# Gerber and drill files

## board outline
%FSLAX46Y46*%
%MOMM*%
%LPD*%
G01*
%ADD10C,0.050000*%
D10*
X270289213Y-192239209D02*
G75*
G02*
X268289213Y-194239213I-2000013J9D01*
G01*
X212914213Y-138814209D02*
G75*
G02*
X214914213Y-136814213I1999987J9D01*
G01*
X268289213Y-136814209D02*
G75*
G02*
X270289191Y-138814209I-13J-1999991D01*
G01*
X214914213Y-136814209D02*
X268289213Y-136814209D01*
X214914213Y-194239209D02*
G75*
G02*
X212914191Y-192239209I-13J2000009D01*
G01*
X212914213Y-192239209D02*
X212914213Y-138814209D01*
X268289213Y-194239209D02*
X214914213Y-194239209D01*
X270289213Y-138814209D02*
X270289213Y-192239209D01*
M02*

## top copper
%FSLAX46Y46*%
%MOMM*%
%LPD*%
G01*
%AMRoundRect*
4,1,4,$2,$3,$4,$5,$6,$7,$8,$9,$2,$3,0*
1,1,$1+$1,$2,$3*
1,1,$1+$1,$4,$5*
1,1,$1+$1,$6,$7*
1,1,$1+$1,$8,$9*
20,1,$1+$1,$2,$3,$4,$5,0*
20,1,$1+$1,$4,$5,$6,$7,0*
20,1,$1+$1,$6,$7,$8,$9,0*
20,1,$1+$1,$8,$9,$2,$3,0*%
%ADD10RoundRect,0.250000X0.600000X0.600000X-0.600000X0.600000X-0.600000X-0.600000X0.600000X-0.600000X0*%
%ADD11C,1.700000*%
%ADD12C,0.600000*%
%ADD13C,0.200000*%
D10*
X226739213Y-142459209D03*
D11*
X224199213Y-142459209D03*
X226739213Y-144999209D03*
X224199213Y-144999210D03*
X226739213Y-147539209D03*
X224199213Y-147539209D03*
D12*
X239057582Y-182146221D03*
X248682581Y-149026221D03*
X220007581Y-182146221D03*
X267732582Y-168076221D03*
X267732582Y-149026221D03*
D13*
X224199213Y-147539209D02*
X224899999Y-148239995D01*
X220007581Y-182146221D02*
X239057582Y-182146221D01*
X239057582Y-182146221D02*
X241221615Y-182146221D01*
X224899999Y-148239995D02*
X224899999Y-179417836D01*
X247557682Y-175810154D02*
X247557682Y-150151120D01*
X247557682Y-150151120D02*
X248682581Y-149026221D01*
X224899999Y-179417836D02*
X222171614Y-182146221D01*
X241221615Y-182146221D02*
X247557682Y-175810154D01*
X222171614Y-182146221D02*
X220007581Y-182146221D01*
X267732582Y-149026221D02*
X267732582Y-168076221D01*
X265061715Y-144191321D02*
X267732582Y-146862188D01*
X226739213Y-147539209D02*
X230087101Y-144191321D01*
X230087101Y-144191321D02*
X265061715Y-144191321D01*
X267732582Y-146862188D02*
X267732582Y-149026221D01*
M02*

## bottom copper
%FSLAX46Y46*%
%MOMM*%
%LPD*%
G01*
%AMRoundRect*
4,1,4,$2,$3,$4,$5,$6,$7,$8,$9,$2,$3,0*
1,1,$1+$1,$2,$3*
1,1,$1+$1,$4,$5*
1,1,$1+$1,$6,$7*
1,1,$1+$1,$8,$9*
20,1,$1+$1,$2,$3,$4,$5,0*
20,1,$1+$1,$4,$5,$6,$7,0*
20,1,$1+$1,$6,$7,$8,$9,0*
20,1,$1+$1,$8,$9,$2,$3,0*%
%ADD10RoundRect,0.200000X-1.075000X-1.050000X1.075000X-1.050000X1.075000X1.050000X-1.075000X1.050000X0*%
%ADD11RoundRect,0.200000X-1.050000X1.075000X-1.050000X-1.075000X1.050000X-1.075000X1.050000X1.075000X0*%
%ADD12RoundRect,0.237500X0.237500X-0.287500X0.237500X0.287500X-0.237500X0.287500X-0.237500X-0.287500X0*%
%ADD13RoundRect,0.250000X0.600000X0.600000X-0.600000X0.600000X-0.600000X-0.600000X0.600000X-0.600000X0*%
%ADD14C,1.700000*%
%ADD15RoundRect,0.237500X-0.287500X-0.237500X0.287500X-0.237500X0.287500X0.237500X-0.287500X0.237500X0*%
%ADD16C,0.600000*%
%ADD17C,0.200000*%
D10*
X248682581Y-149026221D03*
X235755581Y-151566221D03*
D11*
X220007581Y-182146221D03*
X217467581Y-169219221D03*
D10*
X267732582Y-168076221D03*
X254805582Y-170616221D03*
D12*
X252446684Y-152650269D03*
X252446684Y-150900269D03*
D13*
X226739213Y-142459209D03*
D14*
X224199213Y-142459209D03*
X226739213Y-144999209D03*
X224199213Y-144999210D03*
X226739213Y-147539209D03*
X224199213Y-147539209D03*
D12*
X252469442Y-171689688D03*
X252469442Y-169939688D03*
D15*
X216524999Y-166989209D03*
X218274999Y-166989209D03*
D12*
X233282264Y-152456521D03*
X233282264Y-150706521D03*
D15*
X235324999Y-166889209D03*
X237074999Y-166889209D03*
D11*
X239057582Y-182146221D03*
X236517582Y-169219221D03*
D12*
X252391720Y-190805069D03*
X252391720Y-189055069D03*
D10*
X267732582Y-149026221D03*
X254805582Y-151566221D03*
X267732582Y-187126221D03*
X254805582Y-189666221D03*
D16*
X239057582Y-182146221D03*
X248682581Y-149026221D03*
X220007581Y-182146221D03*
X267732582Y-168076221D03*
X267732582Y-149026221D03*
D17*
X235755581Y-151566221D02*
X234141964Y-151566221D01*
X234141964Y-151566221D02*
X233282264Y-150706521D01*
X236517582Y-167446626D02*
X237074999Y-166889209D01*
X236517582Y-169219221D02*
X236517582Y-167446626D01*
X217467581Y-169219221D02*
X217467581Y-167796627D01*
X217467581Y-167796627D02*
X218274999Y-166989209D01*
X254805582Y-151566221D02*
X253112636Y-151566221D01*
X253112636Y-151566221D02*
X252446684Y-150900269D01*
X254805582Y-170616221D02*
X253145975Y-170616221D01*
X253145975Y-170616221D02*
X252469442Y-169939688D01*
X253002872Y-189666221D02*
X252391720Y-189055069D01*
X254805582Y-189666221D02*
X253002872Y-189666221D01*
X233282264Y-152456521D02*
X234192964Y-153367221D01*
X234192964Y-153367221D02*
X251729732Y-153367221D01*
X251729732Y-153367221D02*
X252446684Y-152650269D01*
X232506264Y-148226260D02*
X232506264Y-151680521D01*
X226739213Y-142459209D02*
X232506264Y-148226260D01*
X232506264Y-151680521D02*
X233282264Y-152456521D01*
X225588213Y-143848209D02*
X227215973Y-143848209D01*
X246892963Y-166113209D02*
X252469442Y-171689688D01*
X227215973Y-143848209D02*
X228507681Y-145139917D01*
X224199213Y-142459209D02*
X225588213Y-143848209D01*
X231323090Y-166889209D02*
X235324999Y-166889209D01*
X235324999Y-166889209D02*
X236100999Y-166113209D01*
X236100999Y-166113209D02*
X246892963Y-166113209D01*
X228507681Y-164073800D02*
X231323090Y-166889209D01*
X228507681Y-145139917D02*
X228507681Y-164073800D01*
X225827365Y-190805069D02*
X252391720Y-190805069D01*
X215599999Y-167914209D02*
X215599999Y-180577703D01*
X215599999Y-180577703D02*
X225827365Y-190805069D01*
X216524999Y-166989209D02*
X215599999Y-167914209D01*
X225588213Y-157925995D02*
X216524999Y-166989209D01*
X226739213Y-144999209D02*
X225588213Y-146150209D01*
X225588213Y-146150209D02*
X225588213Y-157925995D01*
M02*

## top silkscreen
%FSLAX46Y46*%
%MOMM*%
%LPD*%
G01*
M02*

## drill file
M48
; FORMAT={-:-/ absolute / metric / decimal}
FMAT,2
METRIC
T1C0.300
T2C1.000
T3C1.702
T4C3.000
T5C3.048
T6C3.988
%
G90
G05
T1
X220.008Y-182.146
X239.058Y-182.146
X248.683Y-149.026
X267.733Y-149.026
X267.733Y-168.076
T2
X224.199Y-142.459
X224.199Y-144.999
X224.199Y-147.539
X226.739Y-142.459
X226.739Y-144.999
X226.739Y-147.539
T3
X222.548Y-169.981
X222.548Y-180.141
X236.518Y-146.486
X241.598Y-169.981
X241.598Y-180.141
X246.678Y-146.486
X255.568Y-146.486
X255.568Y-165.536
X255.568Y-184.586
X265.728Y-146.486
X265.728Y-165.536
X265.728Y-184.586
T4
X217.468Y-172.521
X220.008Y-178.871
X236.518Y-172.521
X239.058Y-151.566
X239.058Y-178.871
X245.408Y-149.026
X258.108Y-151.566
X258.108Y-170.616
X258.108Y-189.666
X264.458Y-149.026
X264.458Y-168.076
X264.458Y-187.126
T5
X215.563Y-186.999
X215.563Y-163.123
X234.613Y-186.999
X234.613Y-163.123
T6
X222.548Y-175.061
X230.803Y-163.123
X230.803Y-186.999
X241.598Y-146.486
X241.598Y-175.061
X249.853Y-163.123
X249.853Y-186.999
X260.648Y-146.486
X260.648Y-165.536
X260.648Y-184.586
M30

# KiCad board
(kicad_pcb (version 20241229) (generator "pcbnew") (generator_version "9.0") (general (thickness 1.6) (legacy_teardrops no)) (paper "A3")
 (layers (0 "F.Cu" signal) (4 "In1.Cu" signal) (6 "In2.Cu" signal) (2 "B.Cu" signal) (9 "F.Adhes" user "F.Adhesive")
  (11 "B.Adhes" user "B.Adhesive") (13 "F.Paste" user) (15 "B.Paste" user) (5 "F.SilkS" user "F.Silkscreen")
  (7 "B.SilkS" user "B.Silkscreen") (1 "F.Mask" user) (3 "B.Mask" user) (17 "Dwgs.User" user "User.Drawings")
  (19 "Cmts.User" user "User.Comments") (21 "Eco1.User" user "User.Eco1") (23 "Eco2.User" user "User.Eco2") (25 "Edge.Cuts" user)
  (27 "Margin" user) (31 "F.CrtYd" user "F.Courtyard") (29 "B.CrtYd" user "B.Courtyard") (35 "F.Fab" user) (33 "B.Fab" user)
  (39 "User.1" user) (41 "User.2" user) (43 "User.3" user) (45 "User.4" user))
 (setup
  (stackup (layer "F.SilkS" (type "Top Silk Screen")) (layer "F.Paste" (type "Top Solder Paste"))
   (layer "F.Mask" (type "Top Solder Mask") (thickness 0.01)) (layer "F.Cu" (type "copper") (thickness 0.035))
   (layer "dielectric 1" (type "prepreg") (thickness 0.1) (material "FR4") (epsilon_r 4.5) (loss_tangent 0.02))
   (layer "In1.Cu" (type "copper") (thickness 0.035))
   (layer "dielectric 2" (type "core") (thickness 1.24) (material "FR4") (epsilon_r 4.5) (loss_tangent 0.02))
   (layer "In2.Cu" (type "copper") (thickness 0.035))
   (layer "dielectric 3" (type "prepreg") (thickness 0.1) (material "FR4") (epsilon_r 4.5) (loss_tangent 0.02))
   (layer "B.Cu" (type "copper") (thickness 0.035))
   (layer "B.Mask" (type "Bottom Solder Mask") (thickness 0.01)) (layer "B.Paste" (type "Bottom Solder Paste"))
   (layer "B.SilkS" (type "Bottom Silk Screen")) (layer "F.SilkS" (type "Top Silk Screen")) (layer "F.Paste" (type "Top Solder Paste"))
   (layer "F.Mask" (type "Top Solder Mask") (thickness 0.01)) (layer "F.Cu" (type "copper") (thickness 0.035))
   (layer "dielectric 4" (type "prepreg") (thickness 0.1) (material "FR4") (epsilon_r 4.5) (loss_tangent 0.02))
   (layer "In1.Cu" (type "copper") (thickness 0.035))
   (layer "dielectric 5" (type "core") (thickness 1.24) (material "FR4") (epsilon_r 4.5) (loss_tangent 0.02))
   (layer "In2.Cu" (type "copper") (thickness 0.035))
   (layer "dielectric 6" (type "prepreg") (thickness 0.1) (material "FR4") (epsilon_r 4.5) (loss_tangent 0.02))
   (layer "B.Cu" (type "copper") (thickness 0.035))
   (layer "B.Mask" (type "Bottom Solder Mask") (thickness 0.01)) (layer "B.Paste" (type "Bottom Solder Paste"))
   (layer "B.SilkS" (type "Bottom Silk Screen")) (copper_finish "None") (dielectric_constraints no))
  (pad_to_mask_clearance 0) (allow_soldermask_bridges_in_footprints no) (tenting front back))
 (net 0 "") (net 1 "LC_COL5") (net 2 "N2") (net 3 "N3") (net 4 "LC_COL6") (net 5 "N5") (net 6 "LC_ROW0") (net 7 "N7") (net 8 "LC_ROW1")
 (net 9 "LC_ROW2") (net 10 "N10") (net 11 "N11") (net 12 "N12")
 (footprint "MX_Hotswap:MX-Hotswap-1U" (layer "B.Cu") (at 241.597581 146.486221)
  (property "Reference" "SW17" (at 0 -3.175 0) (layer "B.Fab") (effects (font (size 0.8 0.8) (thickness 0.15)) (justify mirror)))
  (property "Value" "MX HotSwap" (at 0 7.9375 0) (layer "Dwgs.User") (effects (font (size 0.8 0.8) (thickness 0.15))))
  (pad "" np_thru_hole circle (at -5.08 0 48.099) (size 1.7018 1.7018) (drill 1.7018) (layers "*.Cu" "*.Mask"))
  (pad "" np_thru_hole circle (at -2.54 5.08) (size 3 3) (drill 3) (layers "*.Cu" "*.Mask"))
  (pad "" np_thru_hole circle (at 0 0) (size 3.9878 3.9878) (drill 3.9878) (layers "*.Cu" "*.Mask"))
  (pad "" np_thru_hole circle (at 3.81 2.54) (size 3 3) (drill 3) (layers "*.Cu" "*.Mask"))
  (pad "" np_thru_hole circle (at 5.08 0 48.099) (size 1.7018 1.7018) (drill 1.7018) (layers "*.Cu" "*.Mask"))
  (pad "1" smd roundrect (at 7.085 2.54) (size 2.55 2.5) (layers "B.Cu" "B.Mask" "B.Paste") (roundrect_rratio 0.08) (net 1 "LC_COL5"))
  (pad "2" smd roundrect (at -5.842 5.08) (size 2.55 2.5) (layers "B.Cu" "B.Mask" "B.Paste") (roundrect_rratio 0.08) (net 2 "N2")))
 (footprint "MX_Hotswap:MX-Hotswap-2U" (layer "B.Cu") (at 222.547581 175.061221 -90)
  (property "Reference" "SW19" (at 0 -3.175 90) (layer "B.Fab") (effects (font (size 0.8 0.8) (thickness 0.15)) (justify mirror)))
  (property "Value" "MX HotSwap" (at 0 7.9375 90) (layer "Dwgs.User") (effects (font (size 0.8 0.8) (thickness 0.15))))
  (pad "" np_thru_hole circle (at -11.938 -8.255 270) (size 3.9878 3.9878) (drill 3.9878) (layers "*.Cu" "*.Mask"))
  (pad "" np_thru_hole circle (at -11.938 6.984999 270) (size 3.048 3.048) (drill 3.048) (layers "*.Cu" "*.Mask"))
  (pad "" np_thru_hole circle (at -5.08 0 318.099) (size 1.7018 1.7018) (drill 1.7018) (layers "*.Cu" "*.Mask"))
  (pad "" np_thru_hole circle (at -2.54 5.08 270) (size 3 3) (drill 3) (layers "*.Cu" "*.Mask"))
  (pad "" np_thru_hole circle (at 0 0 270) (size 3.9878 3.9878) (drill 3.9878) (layers "*.Cu" "*.Mask"))
  (pad "" np_thru_hole circle (at 3.81 2.54 270) (size 3 3) (drill 3) (layers "*.Cu" "*.Mask"))
  (pad "" np_thru_hole circle (at 5.08 0 318.099) (size 1.7018 1.7018) (drill 1.7018) (layers "*.Cu" "*.Mask"))
  (pad "" np_thru_hole circle (at 11.938 -8.255 270) (size 3.9878 3.9878) (drill 3.9878) (layers "*.Cu" "*.Mask"))
  (pad "" np_thru_hole circle (at 11.938 6.985 270) (size 3.048 3.048) (drill 3.048) (layers "*.Cu" "*.Mask"))
  (pad "1" smd roundrect (at 7.085 2.54 270) (size 2.55 2.5) (layers "B.Cu" "B.Mask" "B.Paste") (roundrect_rratio 0.08) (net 1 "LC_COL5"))
  (pad "2" smd roundrect (at -5.842 5.08 270) (size 2.55 2.5) (layers "B.Cu" "B.Mask" "B.Paste") (roundrect_rratio 0.08) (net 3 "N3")))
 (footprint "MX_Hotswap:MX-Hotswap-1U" (layer "B.Cu") (at 260.647582 165.536221)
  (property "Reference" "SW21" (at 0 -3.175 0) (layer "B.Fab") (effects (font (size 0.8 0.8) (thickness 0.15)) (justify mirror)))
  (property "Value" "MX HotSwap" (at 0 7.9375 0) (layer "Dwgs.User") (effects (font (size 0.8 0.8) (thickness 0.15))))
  (pad "" np_thru_hole circle (at -5.08 0 48.099) (size 1.7018 1.7018) (drill 1.7018) (layers "*.Cu" "*.Mask"))
  (pad "" np_thru_hole circle (at -2.54 5.08) (size 3 3) (drill 3) (layers "*.Cu" "*.Mask"))
  (pad "" np_thru_hole circle (at 0 0) (size 3.9878 3.9878) (drill 3.9878) (layers "*.Cu" "*.Mask"))
  (pad "" np_thru_hole circle (at 3.81 2.54) (size 3 3) (drill 3) (layers "*.Cu" "*.Mask"))
  (pad "" np_thru_hole circle (at 5.08 0 48.099) (size 1.7018 1.7018) (drill 1.7018) (layers "*.Cu" "*.Mask"))
  (pad "1" smd roundrect (at 7.085 2.54) (size 2.55 2.5) (layers "B.Cu" "B.Mask" "B.Paste") (roundrect_rratio 0.08) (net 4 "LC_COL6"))
  (pad "2" smd roundrect (at -5.842 5.08) (size 2.55 2.5) (layers "B.Cu" "B.Mask" "B.Paste") (roundrect_rratio 0.08) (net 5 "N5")))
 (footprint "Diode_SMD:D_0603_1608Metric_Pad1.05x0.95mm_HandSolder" (layer "B.Cu") (at 252.446684 151.775269 90)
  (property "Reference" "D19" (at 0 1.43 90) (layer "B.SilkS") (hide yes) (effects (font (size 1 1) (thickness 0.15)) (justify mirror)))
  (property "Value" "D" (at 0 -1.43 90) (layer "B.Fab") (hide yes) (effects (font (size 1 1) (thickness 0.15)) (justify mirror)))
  (pad "1" smd roundrect (at -0.875 0 90) (size 1.05 0.95) (layers "B.Cu" "B.Mask" "B.Paste") (roundrect_rratio 0.25) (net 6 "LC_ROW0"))
  (pad "2" smd roundrect (at 0.875 0 90) (size 1.05 0.95) (layers "B.Cu" "B.Mask" "B.Paste") (roundrect_rratio 0.25) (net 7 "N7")))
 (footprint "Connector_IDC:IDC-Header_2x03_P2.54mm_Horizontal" (layer "B.Cu") (at 226.739213 142.459209 180)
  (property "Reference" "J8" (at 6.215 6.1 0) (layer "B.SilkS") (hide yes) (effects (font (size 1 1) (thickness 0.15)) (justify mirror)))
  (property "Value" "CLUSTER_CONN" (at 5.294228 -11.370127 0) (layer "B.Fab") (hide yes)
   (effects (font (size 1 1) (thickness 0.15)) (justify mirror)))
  (pad "1" thru_hole roundrect (at 0 0 180) (size 1.7 1.7) (drill 1) (layers "*.Cu" "*.Mask") (remove_unused_layers no)
   (roundrect_rratio 0.147059) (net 6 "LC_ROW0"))
  (pad "2" thru_hole circle (at 2.54 0 180) (size 1.7 1.7) (drill 1) (layers "*.Cu" "*.Mask") (remove_unused_layers no) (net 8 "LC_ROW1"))
  (pad "3" thru_hole circle (at 0 -2.54 180) (size 1.7 1.7) (drill 1) (layers "*.Cu" "*.Mask") (remove_unused_layers no) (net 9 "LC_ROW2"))
  (pad "4" thru_hole circle (at 2.54 -2.540001 180) (size 1.7 1.7) (drill 1) (layers "*.Cu" "*.Mask") (remove_unused_layers no)
   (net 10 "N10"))
  (pad "5" thru_hole circle (at 0 -5.08 180) (size 1.7 1.7) (drill 1) (layers "*.Cu" "*.Mask") (remove_unused_layers no) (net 4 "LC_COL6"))
  (pad "6" thru_hole circle (at 2.54 -5.08 180) (size 1.7 1.7) (drill 1) (layers "*.Cu" "*.Mask") (remove_unused_layers no)
   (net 1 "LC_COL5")))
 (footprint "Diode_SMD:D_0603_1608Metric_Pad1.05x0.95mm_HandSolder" (layer "B.Cu") (at 252.469442 170.814688 90)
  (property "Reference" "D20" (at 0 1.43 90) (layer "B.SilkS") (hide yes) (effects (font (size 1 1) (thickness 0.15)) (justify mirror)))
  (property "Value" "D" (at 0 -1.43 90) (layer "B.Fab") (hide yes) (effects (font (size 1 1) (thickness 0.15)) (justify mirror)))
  (pad "1" smd roundrect (at -0.875 0 90) (size 1.05 0.95) (layers "B.Cu" "B.Mask" "B.Paste") (roundrect_rratio 0.25) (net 8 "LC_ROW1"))
  (pad "2" smd roundrect (at 0.875 0 90) (size 1.05 0.95) (layers "B.Cu" "B.Mask" "B.Paste") (roundrect_rratio 0.25) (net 5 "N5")))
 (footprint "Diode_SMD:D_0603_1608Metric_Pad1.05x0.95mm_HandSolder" (layer "B.Cu") (at 217.399999 166.989209)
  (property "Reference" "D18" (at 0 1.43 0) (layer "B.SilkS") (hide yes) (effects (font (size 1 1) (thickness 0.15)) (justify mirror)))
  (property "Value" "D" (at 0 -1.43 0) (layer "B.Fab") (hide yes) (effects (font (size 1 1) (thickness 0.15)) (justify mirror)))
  (pad "1" smd roundrect (at -0.875 0) (size 1.05 0.95) (layers "B.Cu" "B.Mask" "B.Paste") (roundrect_rratio 0.25) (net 9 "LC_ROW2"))
  (pad "2" smd roundrect (at 0.875 0) (size 1.05 0.95) (layers "B.Cu" "B.Mask" "B.Paste") (roundrect_rratio 0.25) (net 3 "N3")))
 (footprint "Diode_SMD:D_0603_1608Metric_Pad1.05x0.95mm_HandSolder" (layer "B.Cu") (at 233.282264 151.581521 90)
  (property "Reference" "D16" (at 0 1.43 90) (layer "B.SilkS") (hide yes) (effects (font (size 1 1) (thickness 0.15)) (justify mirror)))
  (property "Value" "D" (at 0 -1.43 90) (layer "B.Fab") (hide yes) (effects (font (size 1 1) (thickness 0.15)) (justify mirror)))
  (pad "1" smd roundrect (at -0.875 0 90) (size 1.05 0.95) (layers "B.Cu" "B.Mask" "B.Paste") (roundrect_rratio 0.25) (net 6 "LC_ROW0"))
  (pad "2" smd roundrect (at 0.875 0 90) (size 1.05 0.95) (layers "B.Cu" "B.Mask" "B.Paste") (roundrect_rratio 0.25) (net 2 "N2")))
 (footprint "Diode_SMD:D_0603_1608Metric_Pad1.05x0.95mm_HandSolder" (layer "B.Cu") (at 236.199999 166.889209)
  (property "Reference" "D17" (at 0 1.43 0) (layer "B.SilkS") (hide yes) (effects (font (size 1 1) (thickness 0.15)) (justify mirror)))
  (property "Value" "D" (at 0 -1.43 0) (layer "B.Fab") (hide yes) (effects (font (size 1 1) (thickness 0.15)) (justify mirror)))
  (pad "1" smd roundrect (at -0.875 0) (size 1.05 0.95) (layers "B.Cu" "B.Mask" "B.Paste") (roundrect_rratio 0.25) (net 8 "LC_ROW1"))
  (pad "2" smd roundrect (at 0.875 0) (size 1.05 0.95) (layers "B.Cu" "B.Mask" "B.Paste") (roundrect_rratio 0.25) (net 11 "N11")))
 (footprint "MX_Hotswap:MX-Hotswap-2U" (layer "B.Cu") (at 241.597582 175.061221 -90)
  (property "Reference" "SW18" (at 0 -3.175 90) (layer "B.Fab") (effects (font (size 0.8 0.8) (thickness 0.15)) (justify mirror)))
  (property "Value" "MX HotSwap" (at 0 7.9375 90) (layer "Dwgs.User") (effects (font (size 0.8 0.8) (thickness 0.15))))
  (pad "" np_thru_hole circle (at -11.938 -8.255 270) (size 3.9878 3.9878) (drill 3.9878) (layers "*.Cu" "*.Mask"))
  (pad "" np_thru_hole circle (at -11.938 6.984999 270) (size 3.048 3.048) (drill 3.048) (layers "*.Cu" "*.Mask"))
  (pad "" np_thru_hole circle (at -5.08 0 318.099) (size 1.7018 1.7018) (drill 1.7018) (layers "*.Cu" "*.Mask"))
  (pad "" np_thru_hole circle (at -2.54 5.08 270) (size 3 3) (drill 3) (layers "*.Cu" "*.Mask"))
  (pad "" np_thru_hole circle (at 0 0 270) (size 3.9878 3.9878) (drill 3.9878) (layers "*.Cu" "*.Mask"))
  (pad "" np_thru_hole circle (at 3.81 2.54 270) (size 3 3) (drill 3) (layers "*.Cu" "*.Mask"))
  (pad "" np_thru_hole circle (at 5.08 0 318.099) (size 1.7018 1.7018) (drill 1.7018) (layers "*.Cu" "*.Mask"))
  (pad "" np_thru_hole circle (at 11.938 -8.255 270) (size 3.9878 3.9878) (drill 3.9878) (layers "*.Cu" "*.Mask"))
  (pad "" np_thru_hole circle (at 11.938 6.985 270) (size 3.048 3.048) (drill 3.048) (layers "*.Cu" "*.Mask"))
  (pad "1" smd roundrect (at 7.085 2.54 270) (size 2.55 2.5) (layers "B.Cu" "B.Mask" "B.Paste") (roundrect_rratio 0.08) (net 1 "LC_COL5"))
  (pad "2" smd roundrect (at -5.842 5.08 270) (size 2.55 2.5) (layers "B.Cu" "B.Mask" "B.Paste") (roundrect_rratio 0.08) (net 11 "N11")))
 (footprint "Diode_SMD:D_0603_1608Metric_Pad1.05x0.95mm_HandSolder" (layer "B.Cu") (at 252.39172 189.930069 90)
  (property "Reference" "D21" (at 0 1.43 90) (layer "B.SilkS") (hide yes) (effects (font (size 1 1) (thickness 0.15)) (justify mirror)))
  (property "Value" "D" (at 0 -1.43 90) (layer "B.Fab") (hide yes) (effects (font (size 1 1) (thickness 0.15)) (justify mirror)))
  (pad "1" smd roundrect (at -0.875 0 90) (size 1.05 0.95) (layers "B.Cu" "B.Mask" "B.Paste") (roundrect_rratio 0.25) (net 9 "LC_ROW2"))
  (pad "2" smd roundrect (at 0.875 0 90) (size 1.05 0.95) (layers "B.Cu" "B.Mask" "B.Paste") (roundrect_rratio 0.25) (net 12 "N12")))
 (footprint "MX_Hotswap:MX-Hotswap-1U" (layer "B.Cu") (at 260.647582 146.486221)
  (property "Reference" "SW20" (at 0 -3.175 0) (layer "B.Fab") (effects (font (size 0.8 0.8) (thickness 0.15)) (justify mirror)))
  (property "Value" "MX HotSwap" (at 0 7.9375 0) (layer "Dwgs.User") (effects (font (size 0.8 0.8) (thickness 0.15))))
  (pad "" np_thru_hole circle (at -5.08 0 48.099) (size 1.7018 1.7018) (drill 1.7018) (layers "*.Cu" "*.Mask"))
  (pad "" np_thru_hole circle (at -2.54 5.08) (size 3 3) (drill 3) (layers "*.Cu" "*.Mask"))
  (pad "" np_thru_hole circle (at 0 0) (size 3.9878 3.9878) (drill 3.9878) (layers "*.Cu" "*.Mask"))
  (pad "" np_thru_hole circle (at 3.81 2.54) (size 3 3) (drill 3) (layers "*.Cu" "*.Mask"))
  (pad "" np_thru_hole circle (at 5.08 0 48.099) (size 1.7018 1.7018) (drill 1.7018) (layers "*.Cu" "*.Mask"))
  (pad "1" smd roundrect (at 7.085 2.54) (size 2.55 2.5) (layers "B.Cu" "B.Mask" "B.Paste") (roundrect_rratio 0.08) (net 4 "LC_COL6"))
  (pad "2" smd roundrect (at -5.842 5.08) (size 2.55 2.5) (layers "B.Cu" "B.Mask" "B.Paste") (roundrect_rratio 0.08) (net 7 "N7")))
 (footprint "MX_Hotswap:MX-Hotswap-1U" (layer "B.Cu") (at 260.647582 184.586221)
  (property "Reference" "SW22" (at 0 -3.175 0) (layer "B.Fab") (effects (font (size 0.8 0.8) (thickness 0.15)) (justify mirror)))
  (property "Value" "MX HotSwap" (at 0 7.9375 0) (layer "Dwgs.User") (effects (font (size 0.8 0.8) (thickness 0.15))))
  (pad "" np_thru_hole circle (at -5.08 0 48.099) (size 1.7018 1.7018) (drill 1.7018) (layers "*.Cu" "*.Mask"))
  (pad "" np_thru_hole circle (at -2.54 5.08) (size 3 3) (drill 3) (layers "*.Cu" "*.Mask"))
  (pad "" np_thru_hole circle (at 0 0) (size 3.9878 3.9878) (drill 3.9878) (layers "*.Cu" "*.Mask"))
  (pad "" np_thru_hole circle (at 3.81 2.54) (size 3 3) (drill 3) (layers "*.Cu" "*.Mask"))
  (pad "" np_thru_hole circle (at 5.08 0 48.099) (size 1.7018 1.7018) (drill 1.7018) (layers "*.Cu" "*.Mask"))
  (pad "1" smd roundrect (at 7.085 2.54) (size 2.55 2.5) (layers "B.Cu" "B.Mask" "B.Paste") (roundrect_rratio 0.08) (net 4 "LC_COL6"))
  (pad "2" smd roundrect (at -5.842 5.08) (size 2.55 2.5) (layers "B.Cu" "B.Mask" "B.Paste") (roundrect_rratio 0.08) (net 12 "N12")))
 (gr_arc (start 270.289213 192.239209) (mid 269.703427 193.653428) (end 268.289213 194.239209) (stroke (width 0.05) (type default))
  (layer "Edge.Cuts"))
 (gr_arc (start 212.914213 138.814209) (mid 213.5 137.4) (end 214.914213 136.814209) (stroke (width 0.05) (type default))
  (layer "Edge.Cuts"))
 (gr_arc (start 268.289213 136.814209) (mid 269.703418 137.4) (end 270.289213 138.814209) (stroke (width 0.05) (type default))
  (layer "Edge.Cuts"))
 (gr_line (start 214.914213 136.814209) (end 268.289213 136.814209) (stroke (width 0.05) (type default)) (layer "Edge.Cuts"))
 (gr_arc (start 214.914213 194.239209) (mid 213.49999 193.653428) (end 212.914213 192.239209) (stroke (width 0.05) (type default))
  (layer "Edge.Cuts"))
 (gr_line (start 212.914213 192.239209) (end 212.914213 138.814209) (stroke (width 0.05) (type default)) (layer "Edge.Cuts"))
 (gr_line (start 268.289213 194.239209) (end 214.914213 194.239209) (stroke (width 0.05) (type default)) (layer "Edge.Cuts"))
 (gr_line (start 270.289213 138.814209) (end 270.289213 192.239209) (stroke (width 0.05) (type default)) (layer "Edge.Cuts"))
 (segment (start 235.755581 151.566221) (end 234.141964 151.566221) (width 0.2) (layer "B.Cu") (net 2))
 (segment (start 234.141964 151.566221) (end 233.282264 150.706521) (width 0.2) (layer "B.Cu") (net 2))
 (segment (start 236.517582 167.446626) (end 237.074999 166.889209) (width 0.2) (layer "B.Cu") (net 11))
 (segment (start 236.517582 169.219221) (end 236.517582 167.446626) (width 0.2) (layer "B.Cu") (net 11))
 (segment (start 217.467581 169.219221) (end 217.467581 167.796627) (width 0.2) (layer "B.Cu") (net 3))
 (segment (start 217.467581 167.796627) (end 218.274999 166.989209) (width 0.2) (layer "B.Cu") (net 3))
 (segment (start 254.805582 151.566221) (end 253.112636 151.566221) (width 0.2) (layer "B.Cu") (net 7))
 (segment (start 253.112636 151.566221) (end 252.446684 150.900269) (width 0.2) (layer "B.Cu") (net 7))
 (segment (start 254.805582 170.616221) (end 253.145975 170.616221) (width 0.2) (layer "B.Cu") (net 5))
 (segment (start 253.145975 170.616221) (end 252.469442 169.939688) (width 0.2) (layer "B.Cu") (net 5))
 (segment (start 253.002872 189.666221) (end 252.39172 189.055069) (width 0.2) (layer "B.Cu") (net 12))
 (segment (start 254.805582 189.666221) (end 253.002872 189.666221) (width 0.2) (layer "B.Cu") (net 12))
 (segment (start 233.282264 152.456521) (end 234.192964 153.367221) (width 0.2) (layer "B.Cu") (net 6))
 (segment (start 234.192964 153.367221) (end 251.729732 153.367221) (width 0.2) (layer "B.Cu") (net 6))
 (segment (start 251.729732 153.367221) (end 252.446684 152.650269) (width 0.2) (layer "B.Cu") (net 6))
 (segment (start 232.506264 148.22626) (end 232.506264 151.680521) (width 0.2) (layer "B.Cu") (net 6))
 (segment (start 226.739213 142.459209) (end 232.506264 148.22626) (width 0.2) (layer "B.Cu") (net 6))
 (segment (start 232.506264 151.680521) (end 233.282264 152.456521) (width 0.2) (layer "B.Cu") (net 6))
 (segment (start 225.588213 143.848209) (end 227.215973 143.848209) (width 0.2) (layer "B.Cu") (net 8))
 (segment (start 246.892963 166.113209) (end 252.469442 171.689688) (width 0.2) (layer "B.Cu") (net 8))
 (segment (start 227.215973 143.848209) (end 228.507681 145.139917) (width 0.2) (layer "B.Cu") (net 8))
 (segment (start 224.199213 142.459209) (end 225.588213 143.848209) (width 0.2) (layer "B.Cu") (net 8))
 (segment (start 231.32309 166.889209) (end 235.324999 166.889209) (width 0.2) (layer "B.Cu") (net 8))
 (segment (start 235.324999 166.889209) (end 236.100999 166.113209) (width 0.2) (layer "B.Cu") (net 8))
 (segment (start 236.100999 166.113209) (end 246.892963 166.113209) (width 0.2) (layer "B.Cu") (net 8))
 (segment (start 228.507681 164.0738) (end 231.32309 166.889209) (width 0.2) (layer "B.Cu") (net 8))
 (segment (start 228.507681 145.139917) (end 228.507681 164.0738) (width 0.2) (layer "B.Cu") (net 8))
 (segment (start 225.827365 190.805069) (end 252.39172 190.805069) (width 0.2) (layer "B.Cu") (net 9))
 (segment (start 215.599999 167.914209) (end 215.599999 180.577703) (width 0.2) (layer "B.Cu") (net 9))
 (segment (start 215.599999 180.577703) (end 225.827365 190.805069) (width 0.2) (layer "B.Cu") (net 9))
 (segment (start 216.524999 166.989209) (end 215.599999 167.914209) (width 0.2) (layer "B.Cu") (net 9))
 (segment (start 225.588213 157.925995) (end 216.524999 166.989209) (width 0.2) (layer "B.Cu") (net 9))
 (segment (start 226.739213 144.999209) (end 225.588213 146.150209) (width 0.2) (layer "B.Cu") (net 9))
 (segment (start 225.588213 146.150209) (end 225.588213 157.925995) (width 0.2) (layer "B.Cu") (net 9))
 (segment (start 224.199213 147.539209) (end 224.899999 148.239995) (width 0.2) (layer "F.Cu") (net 1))
 (segment (start 220.007581 182.146221) (end 239.057582 182.146221) (width 0.2) (layer "F.Cu") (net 1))
 (segment (start 239.057582 182.146221) (end 241.221615 182.146221) (width 0.2) (layer "F.Cu") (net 1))
 (segment (start 224.899999 148.239995) (end 224.899999 179.417836) (width 0.2) (layer "F.Cu") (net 1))
 (segment (start 247.557682 175.810154) (end 247.557682 150.15112) (width 0.2) (layer "F.Cu") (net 1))
 (segment (start 247.557682 150.15112) (end 248.682581 149.026221) (width 0.2) (layer "F.Cu") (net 1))
 (segment (start 224.899999 179.417836) (end 222.171614 182.146221) (width 0.2) (layer "F.Cu") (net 1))
 (segment (start 241.221615 182.146221) (end 247.557682 175.810154) (width 0.2) (layer "F.Cu") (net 1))
 (segment (start 222.171614 182.146221) (end 220.007581 182.146221) (width 0.2) (layer "F.Cu") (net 1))
 (via (at 239.057582 182.146221) (size 0.6) (drill 0.3) (layers "F.Cu" "B.Cu") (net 1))
 (via (at 248.682581 149.026221) (size 0.6) (drill 0.3) (layers "F.Cu" "B.Cu") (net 1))
 (via (at 220.007581 182.146221) (size 0.6) (drill 0.3) (layers "F.Cu" "B.Cu") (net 1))
 (segment (start 267.732582 149.026221) (end 267.732582 168.076221) (width 0.2) (layer "F.Cu") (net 4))
 (segment (start 265.061715 144.191321) (end 267.732582 146.862188) (width 0.2) (layer "F.Cu") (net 4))
 (segment (start 226.739213 147.539209) (end 230.087101 144.191321) (width 0.2) (layer "F.Cu") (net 4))
 (segment (start 230.087101 144.191321) (end 265.061715 144.191321) (width 0.2) (layer "F.Cu") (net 4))
 (segment (start 267.732582 146.862188) (end 267.732582 149.026221) (width 0.2) (layer "F.Cu") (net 4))
 (via (at 267.732582 168.076221) (size 0.6) (drill 0.3) (layers "F.Cu" "B.Cu") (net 4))
 (via (at 267.732582 149.026221) (size 0.6) (drill 0.3) (layers "F.Cu" "B.Cu") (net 4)))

